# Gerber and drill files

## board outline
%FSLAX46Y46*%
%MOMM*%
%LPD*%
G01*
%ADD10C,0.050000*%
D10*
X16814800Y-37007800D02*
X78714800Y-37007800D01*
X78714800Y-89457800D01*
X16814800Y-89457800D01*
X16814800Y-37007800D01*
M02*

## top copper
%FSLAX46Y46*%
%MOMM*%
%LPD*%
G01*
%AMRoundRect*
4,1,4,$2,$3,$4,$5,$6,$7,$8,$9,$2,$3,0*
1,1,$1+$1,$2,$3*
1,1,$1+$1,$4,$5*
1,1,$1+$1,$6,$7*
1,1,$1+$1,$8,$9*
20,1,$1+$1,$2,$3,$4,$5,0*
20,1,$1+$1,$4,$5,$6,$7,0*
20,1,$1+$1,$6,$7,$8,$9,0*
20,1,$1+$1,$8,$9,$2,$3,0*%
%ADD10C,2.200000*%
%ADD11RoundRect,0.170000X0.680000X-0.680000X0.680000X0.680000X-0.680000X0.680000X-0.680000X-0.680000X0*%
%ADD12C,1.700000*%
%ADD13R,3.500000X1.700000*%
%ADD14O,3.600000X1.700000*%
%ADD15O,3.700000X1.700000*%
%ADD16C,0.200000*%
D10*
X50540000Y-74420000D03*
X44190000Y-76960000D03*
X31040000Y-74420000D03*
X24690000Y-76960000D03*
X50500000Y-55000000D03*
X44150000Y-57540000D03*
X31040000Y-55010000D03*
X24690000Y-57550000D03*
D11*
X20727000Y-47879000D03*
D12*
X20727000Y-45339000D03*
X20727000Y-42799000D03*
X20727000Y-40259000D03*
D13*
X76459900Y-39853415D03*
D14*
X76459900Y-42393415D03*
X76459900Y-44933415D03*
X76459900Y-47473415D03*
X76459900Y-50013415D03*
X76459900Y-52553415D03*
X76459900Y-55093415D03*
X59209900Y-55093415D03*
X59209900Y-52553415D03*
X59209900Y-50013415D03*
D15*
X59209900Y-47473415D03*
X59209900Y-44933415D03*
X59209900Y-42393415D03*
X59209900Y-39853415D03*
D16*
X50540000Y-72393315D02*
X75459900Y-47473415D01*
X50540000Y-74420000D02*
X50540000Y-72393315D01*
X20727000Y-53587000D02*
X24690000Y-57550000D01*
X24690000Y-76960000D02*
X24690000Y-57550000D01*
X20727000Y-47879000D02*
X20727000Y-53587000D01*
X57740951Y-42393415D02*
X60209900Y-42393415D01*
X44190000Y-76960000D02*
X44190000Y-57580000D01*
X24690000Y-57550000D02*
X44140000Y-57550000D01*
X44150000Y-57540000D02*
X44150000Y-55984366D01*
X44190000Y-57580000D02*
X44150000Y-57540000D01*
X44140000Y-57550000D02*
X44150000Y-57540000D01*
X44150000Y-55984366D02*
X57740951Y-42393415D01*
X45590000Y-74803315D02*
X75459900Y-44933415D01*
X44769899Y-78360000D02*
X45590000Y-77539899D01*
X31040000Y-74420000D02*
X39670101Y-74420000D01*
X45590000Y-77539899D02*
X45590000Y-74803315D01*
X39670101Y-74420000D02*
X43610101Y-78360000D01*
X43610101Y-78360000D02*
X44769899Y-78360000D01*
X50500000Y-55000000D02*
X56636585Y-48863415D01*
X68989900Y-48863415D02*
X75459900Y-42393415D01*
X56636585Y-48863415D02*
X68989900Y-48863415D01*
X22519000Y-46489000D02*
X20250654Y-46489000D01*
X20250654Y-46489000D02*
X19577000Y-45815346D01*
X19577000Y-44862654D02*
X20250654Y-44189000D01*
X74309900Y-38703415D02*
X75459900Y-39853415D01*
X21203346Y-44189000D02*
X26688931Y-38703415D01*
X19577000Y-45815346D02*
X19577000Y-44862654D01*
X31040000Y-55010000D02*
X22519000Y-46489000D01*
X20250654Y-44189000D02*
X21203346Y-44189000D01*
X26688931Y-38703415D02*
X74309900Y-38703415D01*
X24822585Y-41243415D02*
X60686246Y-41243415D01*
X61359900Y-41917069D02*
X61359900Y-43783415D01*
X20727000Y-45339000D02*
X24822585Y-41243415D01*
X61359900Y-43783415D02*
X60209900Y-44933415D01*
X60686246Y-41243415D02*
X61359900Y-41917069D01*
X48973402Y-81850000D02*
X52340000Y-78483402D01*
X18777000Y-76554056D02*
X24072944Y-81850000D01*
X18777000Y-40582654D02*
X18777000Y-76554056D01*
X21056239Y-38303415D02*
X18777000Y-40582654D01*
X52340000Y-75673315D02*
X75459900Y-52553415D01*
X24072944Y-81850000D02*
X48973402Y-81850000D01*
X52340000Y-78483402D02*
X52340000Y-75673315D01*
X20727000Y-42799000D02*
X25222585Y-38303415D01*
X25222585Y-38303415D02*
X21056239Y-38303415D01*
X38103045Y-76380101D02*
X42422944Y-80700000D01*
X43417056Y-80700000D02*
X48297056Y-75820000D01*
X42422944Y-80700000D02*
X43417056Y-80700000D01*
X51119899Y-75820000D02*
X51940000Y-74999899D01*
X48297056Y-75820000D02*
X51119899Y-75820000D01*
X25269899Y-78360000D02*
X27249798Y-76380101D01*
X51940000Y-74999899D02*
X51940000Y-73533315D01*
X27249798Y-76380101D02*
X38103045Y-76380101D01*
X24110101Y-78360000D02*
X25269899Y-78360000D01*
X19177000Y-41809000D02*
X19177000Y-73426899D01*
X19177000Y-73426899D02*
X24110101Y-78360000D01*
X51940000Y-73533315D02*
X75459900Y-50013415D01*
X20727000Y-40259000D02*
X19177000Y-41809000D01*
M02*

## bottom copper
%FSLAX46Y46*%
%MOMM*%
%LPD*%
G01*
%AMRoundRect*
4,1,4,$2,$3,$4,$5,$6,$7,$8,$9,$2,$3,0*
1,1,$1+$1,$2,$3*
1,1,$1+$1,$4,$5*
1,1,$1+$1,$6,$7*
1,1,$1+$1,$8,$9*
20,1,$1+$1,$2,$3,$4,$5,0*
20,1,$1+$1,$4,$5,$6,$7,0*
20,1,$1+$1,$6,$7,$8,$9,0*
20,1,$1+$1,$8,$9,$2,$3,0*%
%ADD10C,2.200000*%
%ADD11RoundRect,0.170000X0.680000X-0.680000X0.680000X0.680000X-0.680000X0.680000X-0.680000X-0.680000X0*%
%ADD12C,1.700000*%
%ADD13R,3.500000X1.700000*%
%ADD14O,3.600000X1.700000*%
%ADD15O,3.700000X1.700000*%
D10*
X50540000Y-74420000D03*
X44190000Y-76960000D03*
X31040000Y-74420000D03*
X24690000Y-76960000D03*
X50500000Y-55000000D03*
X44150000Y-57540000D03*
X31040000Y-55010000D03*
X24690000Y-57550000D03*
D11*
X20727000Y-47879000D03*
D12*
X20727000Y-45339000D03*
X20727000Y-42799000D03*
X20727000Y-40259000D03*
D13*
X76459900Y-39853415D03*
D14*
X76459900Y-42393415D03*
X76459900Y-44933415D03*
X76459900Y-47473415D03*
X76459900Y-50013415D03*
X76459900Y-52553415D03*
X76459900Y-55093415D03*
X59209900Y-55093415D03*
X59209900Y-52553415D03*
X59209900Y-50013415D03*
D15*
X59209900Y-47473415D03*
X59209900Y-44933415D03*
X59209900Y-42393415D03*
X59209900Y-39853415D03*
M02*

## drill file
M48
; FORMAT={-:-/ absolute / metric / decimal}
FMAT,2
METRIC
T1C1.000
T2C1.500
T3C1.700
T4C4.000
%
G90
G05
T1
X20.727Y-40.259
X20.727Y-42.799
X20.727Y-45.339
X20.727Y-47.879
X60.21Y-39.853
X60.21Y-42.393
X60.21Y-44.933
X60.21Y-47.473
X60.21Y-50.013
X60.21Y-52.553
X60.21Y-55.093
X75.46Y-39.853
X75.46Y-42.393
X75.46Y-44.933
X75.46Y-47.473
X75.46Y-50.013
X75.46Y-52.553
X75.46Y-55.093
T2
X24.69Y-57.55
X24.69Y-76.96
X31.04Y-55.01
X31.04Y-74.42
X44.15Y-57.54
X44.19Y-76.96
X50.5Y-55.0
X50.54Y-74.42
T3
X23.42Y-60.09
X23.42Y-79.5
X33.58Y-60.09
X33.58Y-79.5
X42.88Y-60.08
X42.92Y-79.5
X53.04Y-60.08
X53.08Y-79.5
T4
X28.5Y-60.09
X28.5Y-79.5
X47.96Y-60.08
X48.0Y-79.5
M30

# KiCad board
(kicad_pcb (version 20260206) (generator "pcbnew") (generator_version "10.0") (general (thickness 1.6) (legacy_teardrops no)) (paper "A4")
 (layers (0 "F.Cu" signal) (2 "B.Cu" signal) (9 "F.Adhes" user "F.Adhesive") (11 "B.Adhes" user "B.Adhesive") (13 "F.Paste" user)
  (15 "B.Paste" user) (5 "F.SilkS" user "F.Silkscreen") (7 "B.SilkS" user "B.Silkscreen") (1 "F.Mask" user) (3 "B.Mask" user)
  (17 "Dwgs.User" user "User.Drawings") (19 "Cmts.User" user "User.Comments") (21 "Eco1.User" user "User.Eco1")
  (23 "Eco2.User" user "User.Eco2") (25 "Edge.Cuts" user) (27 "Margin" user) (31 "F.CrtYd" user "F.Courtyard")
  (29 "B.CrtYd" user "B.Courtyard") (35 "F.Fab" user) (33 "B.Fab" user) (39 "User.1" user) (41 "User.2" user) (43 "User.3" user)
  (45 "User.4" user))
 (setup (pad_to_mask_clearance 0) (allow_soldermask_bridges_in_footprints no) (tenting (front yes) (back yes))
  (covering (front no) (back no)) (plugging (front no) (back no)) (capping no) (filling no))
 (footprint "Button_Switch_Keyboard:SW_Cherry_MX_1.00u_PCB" (layer "F.Cu") (at 50.54 74.42)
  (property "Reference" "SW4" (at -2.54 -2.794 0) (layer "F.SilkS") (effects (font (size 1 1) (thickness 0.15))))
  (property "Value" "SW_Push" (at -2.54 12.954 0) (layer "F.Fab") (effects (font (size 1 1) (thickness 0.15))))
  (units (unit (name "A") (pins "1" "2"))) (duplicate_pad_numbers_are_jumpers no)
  (pad "" np_thru_hole circle (at -7.62 5.08) (size 1.7 1.7) (drill 1.7) (layers "*.Cu" "*.Mask"))
  (pad "" np_thru_hole circle (at -2.54 5.08) (size 4 4) (drill 4) (layers "*.Cu" "*.Mask"))
  (pad "" np_thru_hole circle (at 2.54 5.08) (size 1.7 1.7) (drill 1.7) (layers "*.Cu" "*.Mask"))
  (pad "1" thru_hole circle (at 0 0) (size 2.2 2.2) (drill 1.5) (layers "*.Cu" "*.Mask") (remove_unused_layers no)
   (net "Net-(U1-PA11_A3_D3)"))
  (pad "2" thru_hole circle (at -6.35 2.54) (size 2.2 2.2) (drill 1.5) (layers "*.Cu" "*.Mask") (remove_unused_layers no) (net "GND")))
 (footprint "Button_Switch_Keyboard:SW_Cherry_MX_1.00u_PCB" (layer "F.Cu") (at 31.04 74.42)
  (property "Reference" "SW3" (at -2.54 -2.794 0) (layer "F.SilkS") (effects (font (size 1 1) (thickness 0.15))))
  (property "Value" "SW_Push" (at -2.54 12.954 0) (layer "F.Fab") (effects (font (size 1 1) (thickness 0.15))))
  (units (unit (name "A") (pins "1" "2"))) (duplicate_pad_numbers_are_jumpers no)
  (pad "" np_thru_hole circle (at -7.62 5.08) (size 1.7 1.7) (drill 1.7) (layers "*.Cu" "*.Mask"))
  (pad "" np_thru_hole circle (at -2.54 5.08) (size 4 4) (drill 4) (layers "*.Cu" "*.Mask"))
  (pad "" np_thru_hole circle (at 2.54 5.08) (size 1.7 1.7) (drill 1.7) (layers "*.Cu" "*.Mask"))
  (pad "1" thru_hole circle (at 0 0) (size 2.2 2.2) (drill 1.5) (layers "*.Cu" "*.Mask") (remove_unused_layers no)
   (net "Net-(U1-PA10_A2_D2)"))
  (pad "2" thru_hole circle (at -6.35 2.54) (size 2.2 2.2) (drill 1.5) (layers "*.Cu" "*.Mask") (remove_unused_layers no) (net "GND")))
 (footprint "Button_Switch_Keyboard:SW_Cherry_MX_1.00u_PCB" (layer "F.Cu") (at 50.5 55)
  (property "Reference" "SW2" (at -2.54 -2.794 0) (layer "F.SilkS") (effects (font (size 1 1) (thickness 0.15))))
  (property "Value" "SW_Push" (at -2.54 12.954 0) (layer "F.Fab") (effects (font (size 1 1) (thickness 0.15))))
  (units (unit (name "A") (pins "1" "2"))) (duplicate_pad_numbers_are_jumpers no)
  (pad "" np_thru_hole circle (at -7.62 5.08) (size 1.7 1.7) (drill 1.7) (layers "*.Cu" "*.Mask"))
  (pad "" np_thru_hole circle (at -2.54 5.08) (size 4 4) (drill 4) (layers "*.Cu" "*.Mask"))
  (pad "" np_thru_hole circle (at 2.54 5.08) (size 1.7 1.7) (drill 1.7) (layers "*.Cu" "*.Mask"))
  (pad "1" thru_hole circle (at 0 0) (size 2.2 2.2) (drill 1.5) (layers "*.Cu" "*.Mask") (remove_unused_layers no)
   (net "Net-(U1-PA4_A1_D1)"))
  (pad "2" thru_hole circle (at -6.35 2.54) (size 2.2 2.2) (drill 1.5) (layers "*.Cu" "*.Mask") (remove_unused_layers no) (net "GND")))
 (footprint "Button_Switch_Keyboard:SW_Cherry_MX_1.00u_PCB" (layer "F.Cu") (at 31.04 55.01)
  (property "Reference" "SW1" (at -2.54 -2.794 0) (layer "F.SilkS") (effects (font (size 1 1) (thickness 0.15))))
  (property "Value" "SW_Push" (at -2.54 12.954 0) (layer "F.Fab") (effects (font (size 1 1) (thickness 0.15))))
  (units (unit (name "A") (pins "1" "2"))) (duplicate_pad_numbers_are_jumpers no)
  (pad "" np_thru_hole circle (at -7.62 5.08) (size 1.7 1.7) (drill 1.7) (layers "*.Cu" "*.Mask"))
  (pad "" np_thru_hole circle (at -2.54 5.08) (size 4 4) (drill 4) (layers "*.Cu" "*.Mask"))
  (pad "" np_thru_hole circle (at 2.54 5.08) (size 1.7 1.7) (drill 1.7) (layers "*.Cu" "*.Mask"))
  (pad "1" thru_hole circle (at 0 0) (size 2.2 2.2) (drill 1.5) (layers "*.Cu" "*.Mask") (remove_unused_layers no)
   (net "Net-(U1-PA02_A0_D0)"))
  (pad "2" thru_hole circle (at -6.35 2.54) (size 2.2 2.2) (drill 1.5) (layers "*.Cu" "*.Mask") (remove_unused_layers no) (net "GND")))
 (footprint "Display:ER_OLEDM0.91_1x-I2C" (layer "F.Cu") (at 20.727 47.879 90)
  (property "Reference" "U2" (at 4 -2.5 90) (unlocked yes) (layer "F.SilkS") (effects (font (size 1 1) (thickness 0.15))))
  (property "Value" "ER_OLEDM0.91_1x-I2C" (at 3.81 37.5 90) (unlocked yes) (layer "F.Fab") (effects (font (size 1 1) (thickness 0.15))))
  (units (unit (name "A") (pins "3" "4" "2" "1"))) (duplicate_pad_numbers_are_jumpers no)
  (pad "1" thru_hole roundrect (at 0 0 90) (size 1.7 1.7) (drill 1) (layers "*.Cu" "*.Mask") (remove_unused_layers no)
   (roundrect_rratio 0.1) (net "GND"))
  (pad "2" thru_hole circle (at 2.54 0 90) (size 1.7 1.7) (drill 1) (layers "*.Cu" "*.Mask") (remove_unused_layers no) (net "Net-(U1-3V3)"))
  (pad "3" thru_hole circle (at 5.08 0 90) (size 1.7 1.7) (drill 1) (layers "*.Cu" "*.Mask") (remove_unused_layers no)
   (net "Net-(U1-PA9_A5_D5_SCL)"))
  (pad "4" thru_hole circle (at 7.62 0 90) (size 1.7 1.7) (drill 1) (layers "*.Cu" "*.Mask") (remove_unused_layers no)
   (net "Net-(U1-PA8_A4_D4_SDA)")))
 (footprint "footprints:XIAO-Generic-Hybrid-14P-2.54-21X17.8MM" (layer "B.Cu") (at 67.8349 47.473415 180)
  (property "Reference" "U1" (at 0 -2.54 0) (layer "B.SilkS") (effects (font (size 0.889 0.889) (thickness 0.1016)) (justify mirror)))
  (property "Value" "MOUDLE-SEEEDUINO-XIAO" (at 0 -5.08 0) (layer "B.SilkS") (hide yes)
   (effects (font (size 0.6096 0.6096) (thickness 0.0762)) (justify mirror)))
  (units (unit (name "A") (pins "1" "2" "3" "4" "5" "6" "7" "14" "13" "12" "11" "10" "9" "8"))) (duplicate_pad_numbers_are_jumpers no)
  (pad "1" thru_hole rect (at -7.625 7.62 180) (size 3.5 1.7) (drill 1 (offset -1 0)) (layers "*.Cu" "*.Mask") (remove_unused_layers no)
   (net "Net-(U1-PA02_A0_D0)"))
  (pad "2" thru_hole oval (at -7.625 5.08 180) (size 3.6 1.7) (drill 1 (offset -1 0)) (layers "*.Cu" "*.Mask") (remove_unused_layers no)
   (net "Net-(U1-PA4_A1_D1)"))
  (pad "3" thru_hole oval (at -7.625 2.54 180) (size 3.6 1.7) (drill 1 (offset -1 0)) (layers "*.Cu" "*.Mask") (remove_unused_layers no)
   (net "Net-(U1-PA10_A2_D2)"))
  (pad "4" thru_hole oval (at -7.625 0 180) (size 3.6 1.7) (drill 1 (offset -1 0)) (layers "*.Cu" "*.Mask") (remove_unused_layers no)
   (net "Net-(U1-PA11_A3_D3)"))
  (pad "5" thru_hole oval (at -7.625 -2.54 180) (size 3.6 1.7) (drill 1 (offset -1 0)) (layers "*.Cu" "*.Mask") (remove_unused_layers no)
   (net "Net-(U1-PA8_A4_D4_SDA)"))
  (pad "6" thru_hole oval (at -7.625 -5.08) (size 3.6 1.7) (drill 1 (offset 1 0)) (layers "*.Cu" "*.Mask") (remove_unused_layers no)
   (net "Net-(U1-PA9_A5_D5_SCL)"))
  (pad "7" thru_hole oval (at -7.625 -7.62 180) (size 3.6 1.7) (drill 1 (offset -1 0)) (layers "*.Cu" "*.Mask") (remove_unused_layers no)
   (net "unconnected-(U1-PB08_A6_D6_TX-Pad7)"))
  (pad "8" thru_hole oval (at 7.625 -7.62 180) (size 3.6 1.7) (drill 1 (offset 1 0)) (layers "*.Cu" "*.Mask") (remove_unused_layers no)
   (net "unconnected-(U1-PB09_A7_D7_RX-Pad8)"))
  (pad "9" thru_hole oval (at 7.625 -5.08 180) (size 3.6 1.7) (drill 1 (offset 1 0)) (layers "*.Cu" "*.Mask") (remove_unused_layers no)
   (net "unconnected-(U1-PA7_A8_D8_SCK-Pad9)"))
  (pad "10" thru_hole oval (at 7.625 -2.54 180) (size 3.6 1.7) (drill 1 (offset 1 0)) (layers "*.Cu" "*.Mask") (remove_unused_layers no)
   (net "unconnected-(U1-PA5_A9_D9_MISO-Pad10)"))
  (pad "11" thru_hole oval (at 7.625 0 180) (size 3.7 1.7) (drill 1 (offset 1 0)) (layers "*.Cu" "*.Mask") (remove_unused_layers no)
   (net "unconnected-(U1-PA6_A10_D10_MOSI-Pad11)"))
  (pad "12" thru_hole oval (at 7.625 2.54 180) (size 3.7 1.7) (drill 1 (offset 1 0)) (layers "*.Cu" "*.Mask") (remove_unused_layers no)
   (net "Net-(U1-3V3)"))
  (pad "13" thru_hole oval (at 7.625 5.08 180) (size 3.7 1.7) (drill 1 (offset 1 0)) (layers "*.Cu" "*.Mask") (remove_unused_layers no)
   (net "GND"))
  (pad "14" thru_hole oval (at 7.625 7.62 180) (size 3.7 1.7) (drill 1 (offset 1 0)) (layers "*.Cu" "*.Mask") (remove_unused_layers no)
   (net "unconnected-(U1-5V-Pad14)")))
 (gr_rect (start 16.8148 37.0078) (end 78.7148 89.4578) (stroke (width 0.05) (type default)) (fill no) (layer "Edge.Cuts"))
 (segment (start 50.54 72.393315) (end 75.4599 47.473415) (width 0.2) (layer "F.Cu") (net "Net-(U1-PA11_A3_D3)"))
 (segment (start 50.54 74.42) (end 50.54 72.393315) (width 0.2) (layer "F.Cu") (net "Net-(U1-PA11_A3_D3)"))
 (segment (start 20.727 53.587) (end 24.69 57.55) (width 0.2) (layer "F.Cu") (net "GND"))
 (segment (start 24.69 76.96) (end 24.69 57.55) (width 0.2) (layer "F.Cu") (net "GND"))
 (segment (start 20.727 47.879) (end 20.727 53.587) (width 0.2) (layer "F.Cu") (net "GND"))
 (segment (start 57.740951 42.393415) (end 60.2099 42.393415) (width 0.2) (layer "F.Cu") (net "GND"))
 (segment (start 44.19 76.96) (end 44.19 57.58) (width 0.2) (layer "F.Cu") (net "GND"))
 (segment (start 24.69 57.55) (end 44.14 57.55) (width 0.2) (layer "F.Cu") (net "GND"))
 (segment (start 44.15 57.54) (end 44.15 55.984366) (width 0.2) (layer "F.Cu") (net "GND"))
 (segment (start 44.19 57.58) (end 44.15 57.54) (width 0.2) (layer "F.Cu") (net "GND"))
 (segment (start 44.14 57.55) (end 44.15 57.54) (width 0.2) (layer "F.Cu") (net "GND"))
 (segment (start 44.15 55.984366) (end 57.740951 42.393415) (width 0.2) (layer "F.Cu") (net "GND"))
 (segment (start 45.59 74.803315) (end 75.4599 44.933415) (width 0.2) (layer "F.Cu") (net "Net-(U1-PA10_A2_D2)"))
 (segment (start 44.769899 78.36) (end 45.59 77.539899) (width 0.2) (layer "F.Cu") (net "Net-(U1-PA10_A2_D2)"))
 (segment (start 31.04 74.42) (end 39.670101 74.42) (width 0.2) (layer "F.Cu") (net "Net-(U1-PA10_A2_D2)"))
 (segment (start 45.59 77.539899) (end 45.59 74.803315) (width 0.2) (layer "F.Cu") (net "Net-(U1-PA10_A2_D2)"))
 (segment (start 39.670101 74.42) (end 43.610101 78.36) (width 0.2) (layer "F.Cu") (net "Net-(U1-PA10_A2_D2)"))
 (segment (start 43.610101 78.36) (end 44.769899 78.36) (width 0.2) (layer "F.Cu") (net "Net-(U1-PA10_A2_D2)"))
 (segment (start 50.5 55) (end 56.636585 48.863415) (width 0.2) (layer "F.Cu") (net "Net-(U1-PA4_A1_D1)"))
 (segment (start 68.9899 48.863415) (end 75.4599 42.393415) (width 0.2) (layer "F.Cu") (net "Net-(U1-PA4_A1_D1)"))
 (segment (start 56.636585 48.863415) (end 68.9899 48.863415) (width 0.2) (layer "F.Cu") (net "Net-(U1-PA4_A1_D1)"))
 (segment (start 22.519 46.489) (end 20.250654 46.489) (width 0.2) (layer "F.Cu") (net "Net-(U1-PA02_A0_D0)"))
 (segment (start 20.250654 46.489) (end 19.577 45.815346) (width 0.2) (layer "F.Cu") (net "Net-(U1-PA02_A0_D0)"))
 (segment (start 19.577 44.862654) (end 20.250654 44.189) (width 0.2) (layer "F.Cu") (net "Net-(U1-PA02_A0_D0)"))
 (segment (start 74.3099 38.703415) (end 75.4599 39.853415) (width 0.2) (layer "F.Cu") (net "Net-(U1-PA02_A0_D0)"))
 (segment (start 21.203346 44.189) (end 26.688931 38.703415) (width 0.2) (layer "F.Cu") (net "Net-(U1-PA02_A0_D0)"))
 (segment (start 19.577 45.815346) (end 19.577 44.862654) (width 0.2) (layer "F.Cu") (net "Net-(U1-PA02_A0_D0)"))
 (segment (start 31.04 55.01) (end 22.519 46.489) (width 0.2) (layer "F.Cu") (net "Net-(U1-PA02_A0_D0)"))
 (segment (start 20.250654 44.189) (end 21.203346 44.189) (width 0.2) (layer "F.Cu") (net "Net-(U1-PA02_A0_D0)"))
 (segment (start 26.688931 38.703415) (end 74.3099 38.703415) (width 0.2) (layer "F.Cu") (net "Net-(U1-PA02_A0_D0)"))
 (segment (start 24.822585 41.243415) (end 60.686246 41.243415) (width 0.2) (layer "F.Cu") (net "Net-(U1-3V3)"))
 (segment (start 61.3599 41.917069) (end 61.3599 43.783415) (width 0.2) (layer "F.Cu") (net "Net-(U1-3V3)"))
 (segment (start 20.727 45.339) (end 24.822585 41.243415) (width 0.2) (layer "F.Cu") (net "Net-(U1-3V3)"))
 (segment (start 61.3599 43.783415) (end 60.2099 44.933415) (width 0.2) (layer "F.Cu") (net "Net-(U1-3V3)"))
 (segment (start 60.686246 41.243415) (end 61.3599 41.917069) (width 0.2) (layer "F.Cu") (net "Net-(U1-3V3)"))
 (segment (start 48.973402 81.85) (end 52.34 78.483402) (width 0.2) (layer "F.Cu") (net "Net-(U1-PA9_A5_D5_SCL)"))
 (segment (start 18.777 76.554056) (end 24.072944 81.85) (width 0.2) (layer "F.Cu") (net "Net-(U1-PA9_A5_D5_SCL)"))
 (segment (start 18.777 40.582654) (end 18.777 76.554056) (width 0.2) (layer "F.Cu") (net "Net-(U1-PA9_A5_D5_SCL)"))
 (segment (start 21.056239 38.303415) (end 18.777 40.582654) (width 0.2) (layer "F.Cu") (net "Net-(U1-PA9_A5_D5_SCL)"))
 (segment (start 52.34 75.673315) (end 75.4599 52.553415) (width 0.2) (layer "F.Cu") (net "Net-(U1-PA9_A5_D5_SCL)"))
 (segment (start 24.072944 81.85) (end 48.973402 81.85) (width 0.2) (layer "F.Cu") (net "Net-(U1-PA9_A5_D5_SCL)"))
 (segment (start 52.34 78.483402) (end 52.34 75.673315) (width 0.2) (layer "F.Cu") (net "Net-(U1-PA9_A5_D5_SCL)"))
 (segment (start 20.727 42.799) (end 25.222585 38.303415) (width 0.2) (layer "F.Cu") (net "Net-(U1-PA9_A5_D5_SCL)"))
 (segment (start 25.222585 38.303415) (end 21.056239 38.303415) (width 0.2) (layer "F.Cu") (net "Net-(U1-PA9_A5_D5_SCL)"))
 (segment (start 38.103045 76.380101) (end 42.422944 80.7) (width 0.2) (layer "F.Cu") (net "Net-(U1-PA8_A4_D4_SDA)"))
 (segment (start 43.417056 80.7) (end 48.297056 75.82) (width 0.2) (layer "F.Cu") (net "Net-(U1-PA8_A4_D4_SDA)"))
 (segment (start 42.422944 80.7) (end 43.417056 80.7) (width 0.2) (layer "F.Cu") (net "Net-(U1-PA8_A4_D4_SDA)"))
 (segment (start 51.119899 75.82) (end 51.94 74.999899) (width 0.2) (layer "F.Cu") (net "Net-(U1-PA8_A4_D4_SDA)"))
 (segment (start 48.297056 75.82) (end 51.119899 75.82) (width 0.2) (layer "F.Cu") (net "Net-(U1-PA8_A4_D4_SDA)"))
 (segment (start 25.269899 78.36) (end 27.249798 76.380101) (width 0.2) (layer "F.Cu") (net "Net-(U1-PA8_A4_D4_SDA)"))
 (segment (start 51.94 74.999899) (end 51.94 73.533315) (width 0.2) (layer "F.Cu") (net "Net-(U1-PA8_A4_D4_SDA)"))
 (segment (start 27.249798 76.380101) (end 38.103045 76.380101) (width 0.2) (layer "F.Cu") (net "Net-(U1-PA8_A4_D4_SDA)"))
 (segment (start 24.110101 78.36) (end 25.269899 78.36) (width 0.2) (layer "F.Cu") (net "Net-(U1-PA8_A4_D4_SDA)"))
 (segment (start 19.177 41.809) (end 19.177 73.426899) (width 0.2) (layer "F.Cu") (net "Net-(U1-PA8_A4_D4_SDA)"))
 (segment (start 19.177 73.426899) (end 24.110101 78.36) (width 0.2) (layer "F.Cu") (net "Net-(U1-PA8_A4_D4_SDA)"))
 (segment (start 51.94 73.533315) (end 75.4599 50.013415) (width 0.2) (layer "F.Cu") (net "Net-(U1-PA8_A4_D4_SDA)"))
 (segment (start 20.727 40.259) (end 19.177 41.809) (width 0.2) (layer "F.Cu") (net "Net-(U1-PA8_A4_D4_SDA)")))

